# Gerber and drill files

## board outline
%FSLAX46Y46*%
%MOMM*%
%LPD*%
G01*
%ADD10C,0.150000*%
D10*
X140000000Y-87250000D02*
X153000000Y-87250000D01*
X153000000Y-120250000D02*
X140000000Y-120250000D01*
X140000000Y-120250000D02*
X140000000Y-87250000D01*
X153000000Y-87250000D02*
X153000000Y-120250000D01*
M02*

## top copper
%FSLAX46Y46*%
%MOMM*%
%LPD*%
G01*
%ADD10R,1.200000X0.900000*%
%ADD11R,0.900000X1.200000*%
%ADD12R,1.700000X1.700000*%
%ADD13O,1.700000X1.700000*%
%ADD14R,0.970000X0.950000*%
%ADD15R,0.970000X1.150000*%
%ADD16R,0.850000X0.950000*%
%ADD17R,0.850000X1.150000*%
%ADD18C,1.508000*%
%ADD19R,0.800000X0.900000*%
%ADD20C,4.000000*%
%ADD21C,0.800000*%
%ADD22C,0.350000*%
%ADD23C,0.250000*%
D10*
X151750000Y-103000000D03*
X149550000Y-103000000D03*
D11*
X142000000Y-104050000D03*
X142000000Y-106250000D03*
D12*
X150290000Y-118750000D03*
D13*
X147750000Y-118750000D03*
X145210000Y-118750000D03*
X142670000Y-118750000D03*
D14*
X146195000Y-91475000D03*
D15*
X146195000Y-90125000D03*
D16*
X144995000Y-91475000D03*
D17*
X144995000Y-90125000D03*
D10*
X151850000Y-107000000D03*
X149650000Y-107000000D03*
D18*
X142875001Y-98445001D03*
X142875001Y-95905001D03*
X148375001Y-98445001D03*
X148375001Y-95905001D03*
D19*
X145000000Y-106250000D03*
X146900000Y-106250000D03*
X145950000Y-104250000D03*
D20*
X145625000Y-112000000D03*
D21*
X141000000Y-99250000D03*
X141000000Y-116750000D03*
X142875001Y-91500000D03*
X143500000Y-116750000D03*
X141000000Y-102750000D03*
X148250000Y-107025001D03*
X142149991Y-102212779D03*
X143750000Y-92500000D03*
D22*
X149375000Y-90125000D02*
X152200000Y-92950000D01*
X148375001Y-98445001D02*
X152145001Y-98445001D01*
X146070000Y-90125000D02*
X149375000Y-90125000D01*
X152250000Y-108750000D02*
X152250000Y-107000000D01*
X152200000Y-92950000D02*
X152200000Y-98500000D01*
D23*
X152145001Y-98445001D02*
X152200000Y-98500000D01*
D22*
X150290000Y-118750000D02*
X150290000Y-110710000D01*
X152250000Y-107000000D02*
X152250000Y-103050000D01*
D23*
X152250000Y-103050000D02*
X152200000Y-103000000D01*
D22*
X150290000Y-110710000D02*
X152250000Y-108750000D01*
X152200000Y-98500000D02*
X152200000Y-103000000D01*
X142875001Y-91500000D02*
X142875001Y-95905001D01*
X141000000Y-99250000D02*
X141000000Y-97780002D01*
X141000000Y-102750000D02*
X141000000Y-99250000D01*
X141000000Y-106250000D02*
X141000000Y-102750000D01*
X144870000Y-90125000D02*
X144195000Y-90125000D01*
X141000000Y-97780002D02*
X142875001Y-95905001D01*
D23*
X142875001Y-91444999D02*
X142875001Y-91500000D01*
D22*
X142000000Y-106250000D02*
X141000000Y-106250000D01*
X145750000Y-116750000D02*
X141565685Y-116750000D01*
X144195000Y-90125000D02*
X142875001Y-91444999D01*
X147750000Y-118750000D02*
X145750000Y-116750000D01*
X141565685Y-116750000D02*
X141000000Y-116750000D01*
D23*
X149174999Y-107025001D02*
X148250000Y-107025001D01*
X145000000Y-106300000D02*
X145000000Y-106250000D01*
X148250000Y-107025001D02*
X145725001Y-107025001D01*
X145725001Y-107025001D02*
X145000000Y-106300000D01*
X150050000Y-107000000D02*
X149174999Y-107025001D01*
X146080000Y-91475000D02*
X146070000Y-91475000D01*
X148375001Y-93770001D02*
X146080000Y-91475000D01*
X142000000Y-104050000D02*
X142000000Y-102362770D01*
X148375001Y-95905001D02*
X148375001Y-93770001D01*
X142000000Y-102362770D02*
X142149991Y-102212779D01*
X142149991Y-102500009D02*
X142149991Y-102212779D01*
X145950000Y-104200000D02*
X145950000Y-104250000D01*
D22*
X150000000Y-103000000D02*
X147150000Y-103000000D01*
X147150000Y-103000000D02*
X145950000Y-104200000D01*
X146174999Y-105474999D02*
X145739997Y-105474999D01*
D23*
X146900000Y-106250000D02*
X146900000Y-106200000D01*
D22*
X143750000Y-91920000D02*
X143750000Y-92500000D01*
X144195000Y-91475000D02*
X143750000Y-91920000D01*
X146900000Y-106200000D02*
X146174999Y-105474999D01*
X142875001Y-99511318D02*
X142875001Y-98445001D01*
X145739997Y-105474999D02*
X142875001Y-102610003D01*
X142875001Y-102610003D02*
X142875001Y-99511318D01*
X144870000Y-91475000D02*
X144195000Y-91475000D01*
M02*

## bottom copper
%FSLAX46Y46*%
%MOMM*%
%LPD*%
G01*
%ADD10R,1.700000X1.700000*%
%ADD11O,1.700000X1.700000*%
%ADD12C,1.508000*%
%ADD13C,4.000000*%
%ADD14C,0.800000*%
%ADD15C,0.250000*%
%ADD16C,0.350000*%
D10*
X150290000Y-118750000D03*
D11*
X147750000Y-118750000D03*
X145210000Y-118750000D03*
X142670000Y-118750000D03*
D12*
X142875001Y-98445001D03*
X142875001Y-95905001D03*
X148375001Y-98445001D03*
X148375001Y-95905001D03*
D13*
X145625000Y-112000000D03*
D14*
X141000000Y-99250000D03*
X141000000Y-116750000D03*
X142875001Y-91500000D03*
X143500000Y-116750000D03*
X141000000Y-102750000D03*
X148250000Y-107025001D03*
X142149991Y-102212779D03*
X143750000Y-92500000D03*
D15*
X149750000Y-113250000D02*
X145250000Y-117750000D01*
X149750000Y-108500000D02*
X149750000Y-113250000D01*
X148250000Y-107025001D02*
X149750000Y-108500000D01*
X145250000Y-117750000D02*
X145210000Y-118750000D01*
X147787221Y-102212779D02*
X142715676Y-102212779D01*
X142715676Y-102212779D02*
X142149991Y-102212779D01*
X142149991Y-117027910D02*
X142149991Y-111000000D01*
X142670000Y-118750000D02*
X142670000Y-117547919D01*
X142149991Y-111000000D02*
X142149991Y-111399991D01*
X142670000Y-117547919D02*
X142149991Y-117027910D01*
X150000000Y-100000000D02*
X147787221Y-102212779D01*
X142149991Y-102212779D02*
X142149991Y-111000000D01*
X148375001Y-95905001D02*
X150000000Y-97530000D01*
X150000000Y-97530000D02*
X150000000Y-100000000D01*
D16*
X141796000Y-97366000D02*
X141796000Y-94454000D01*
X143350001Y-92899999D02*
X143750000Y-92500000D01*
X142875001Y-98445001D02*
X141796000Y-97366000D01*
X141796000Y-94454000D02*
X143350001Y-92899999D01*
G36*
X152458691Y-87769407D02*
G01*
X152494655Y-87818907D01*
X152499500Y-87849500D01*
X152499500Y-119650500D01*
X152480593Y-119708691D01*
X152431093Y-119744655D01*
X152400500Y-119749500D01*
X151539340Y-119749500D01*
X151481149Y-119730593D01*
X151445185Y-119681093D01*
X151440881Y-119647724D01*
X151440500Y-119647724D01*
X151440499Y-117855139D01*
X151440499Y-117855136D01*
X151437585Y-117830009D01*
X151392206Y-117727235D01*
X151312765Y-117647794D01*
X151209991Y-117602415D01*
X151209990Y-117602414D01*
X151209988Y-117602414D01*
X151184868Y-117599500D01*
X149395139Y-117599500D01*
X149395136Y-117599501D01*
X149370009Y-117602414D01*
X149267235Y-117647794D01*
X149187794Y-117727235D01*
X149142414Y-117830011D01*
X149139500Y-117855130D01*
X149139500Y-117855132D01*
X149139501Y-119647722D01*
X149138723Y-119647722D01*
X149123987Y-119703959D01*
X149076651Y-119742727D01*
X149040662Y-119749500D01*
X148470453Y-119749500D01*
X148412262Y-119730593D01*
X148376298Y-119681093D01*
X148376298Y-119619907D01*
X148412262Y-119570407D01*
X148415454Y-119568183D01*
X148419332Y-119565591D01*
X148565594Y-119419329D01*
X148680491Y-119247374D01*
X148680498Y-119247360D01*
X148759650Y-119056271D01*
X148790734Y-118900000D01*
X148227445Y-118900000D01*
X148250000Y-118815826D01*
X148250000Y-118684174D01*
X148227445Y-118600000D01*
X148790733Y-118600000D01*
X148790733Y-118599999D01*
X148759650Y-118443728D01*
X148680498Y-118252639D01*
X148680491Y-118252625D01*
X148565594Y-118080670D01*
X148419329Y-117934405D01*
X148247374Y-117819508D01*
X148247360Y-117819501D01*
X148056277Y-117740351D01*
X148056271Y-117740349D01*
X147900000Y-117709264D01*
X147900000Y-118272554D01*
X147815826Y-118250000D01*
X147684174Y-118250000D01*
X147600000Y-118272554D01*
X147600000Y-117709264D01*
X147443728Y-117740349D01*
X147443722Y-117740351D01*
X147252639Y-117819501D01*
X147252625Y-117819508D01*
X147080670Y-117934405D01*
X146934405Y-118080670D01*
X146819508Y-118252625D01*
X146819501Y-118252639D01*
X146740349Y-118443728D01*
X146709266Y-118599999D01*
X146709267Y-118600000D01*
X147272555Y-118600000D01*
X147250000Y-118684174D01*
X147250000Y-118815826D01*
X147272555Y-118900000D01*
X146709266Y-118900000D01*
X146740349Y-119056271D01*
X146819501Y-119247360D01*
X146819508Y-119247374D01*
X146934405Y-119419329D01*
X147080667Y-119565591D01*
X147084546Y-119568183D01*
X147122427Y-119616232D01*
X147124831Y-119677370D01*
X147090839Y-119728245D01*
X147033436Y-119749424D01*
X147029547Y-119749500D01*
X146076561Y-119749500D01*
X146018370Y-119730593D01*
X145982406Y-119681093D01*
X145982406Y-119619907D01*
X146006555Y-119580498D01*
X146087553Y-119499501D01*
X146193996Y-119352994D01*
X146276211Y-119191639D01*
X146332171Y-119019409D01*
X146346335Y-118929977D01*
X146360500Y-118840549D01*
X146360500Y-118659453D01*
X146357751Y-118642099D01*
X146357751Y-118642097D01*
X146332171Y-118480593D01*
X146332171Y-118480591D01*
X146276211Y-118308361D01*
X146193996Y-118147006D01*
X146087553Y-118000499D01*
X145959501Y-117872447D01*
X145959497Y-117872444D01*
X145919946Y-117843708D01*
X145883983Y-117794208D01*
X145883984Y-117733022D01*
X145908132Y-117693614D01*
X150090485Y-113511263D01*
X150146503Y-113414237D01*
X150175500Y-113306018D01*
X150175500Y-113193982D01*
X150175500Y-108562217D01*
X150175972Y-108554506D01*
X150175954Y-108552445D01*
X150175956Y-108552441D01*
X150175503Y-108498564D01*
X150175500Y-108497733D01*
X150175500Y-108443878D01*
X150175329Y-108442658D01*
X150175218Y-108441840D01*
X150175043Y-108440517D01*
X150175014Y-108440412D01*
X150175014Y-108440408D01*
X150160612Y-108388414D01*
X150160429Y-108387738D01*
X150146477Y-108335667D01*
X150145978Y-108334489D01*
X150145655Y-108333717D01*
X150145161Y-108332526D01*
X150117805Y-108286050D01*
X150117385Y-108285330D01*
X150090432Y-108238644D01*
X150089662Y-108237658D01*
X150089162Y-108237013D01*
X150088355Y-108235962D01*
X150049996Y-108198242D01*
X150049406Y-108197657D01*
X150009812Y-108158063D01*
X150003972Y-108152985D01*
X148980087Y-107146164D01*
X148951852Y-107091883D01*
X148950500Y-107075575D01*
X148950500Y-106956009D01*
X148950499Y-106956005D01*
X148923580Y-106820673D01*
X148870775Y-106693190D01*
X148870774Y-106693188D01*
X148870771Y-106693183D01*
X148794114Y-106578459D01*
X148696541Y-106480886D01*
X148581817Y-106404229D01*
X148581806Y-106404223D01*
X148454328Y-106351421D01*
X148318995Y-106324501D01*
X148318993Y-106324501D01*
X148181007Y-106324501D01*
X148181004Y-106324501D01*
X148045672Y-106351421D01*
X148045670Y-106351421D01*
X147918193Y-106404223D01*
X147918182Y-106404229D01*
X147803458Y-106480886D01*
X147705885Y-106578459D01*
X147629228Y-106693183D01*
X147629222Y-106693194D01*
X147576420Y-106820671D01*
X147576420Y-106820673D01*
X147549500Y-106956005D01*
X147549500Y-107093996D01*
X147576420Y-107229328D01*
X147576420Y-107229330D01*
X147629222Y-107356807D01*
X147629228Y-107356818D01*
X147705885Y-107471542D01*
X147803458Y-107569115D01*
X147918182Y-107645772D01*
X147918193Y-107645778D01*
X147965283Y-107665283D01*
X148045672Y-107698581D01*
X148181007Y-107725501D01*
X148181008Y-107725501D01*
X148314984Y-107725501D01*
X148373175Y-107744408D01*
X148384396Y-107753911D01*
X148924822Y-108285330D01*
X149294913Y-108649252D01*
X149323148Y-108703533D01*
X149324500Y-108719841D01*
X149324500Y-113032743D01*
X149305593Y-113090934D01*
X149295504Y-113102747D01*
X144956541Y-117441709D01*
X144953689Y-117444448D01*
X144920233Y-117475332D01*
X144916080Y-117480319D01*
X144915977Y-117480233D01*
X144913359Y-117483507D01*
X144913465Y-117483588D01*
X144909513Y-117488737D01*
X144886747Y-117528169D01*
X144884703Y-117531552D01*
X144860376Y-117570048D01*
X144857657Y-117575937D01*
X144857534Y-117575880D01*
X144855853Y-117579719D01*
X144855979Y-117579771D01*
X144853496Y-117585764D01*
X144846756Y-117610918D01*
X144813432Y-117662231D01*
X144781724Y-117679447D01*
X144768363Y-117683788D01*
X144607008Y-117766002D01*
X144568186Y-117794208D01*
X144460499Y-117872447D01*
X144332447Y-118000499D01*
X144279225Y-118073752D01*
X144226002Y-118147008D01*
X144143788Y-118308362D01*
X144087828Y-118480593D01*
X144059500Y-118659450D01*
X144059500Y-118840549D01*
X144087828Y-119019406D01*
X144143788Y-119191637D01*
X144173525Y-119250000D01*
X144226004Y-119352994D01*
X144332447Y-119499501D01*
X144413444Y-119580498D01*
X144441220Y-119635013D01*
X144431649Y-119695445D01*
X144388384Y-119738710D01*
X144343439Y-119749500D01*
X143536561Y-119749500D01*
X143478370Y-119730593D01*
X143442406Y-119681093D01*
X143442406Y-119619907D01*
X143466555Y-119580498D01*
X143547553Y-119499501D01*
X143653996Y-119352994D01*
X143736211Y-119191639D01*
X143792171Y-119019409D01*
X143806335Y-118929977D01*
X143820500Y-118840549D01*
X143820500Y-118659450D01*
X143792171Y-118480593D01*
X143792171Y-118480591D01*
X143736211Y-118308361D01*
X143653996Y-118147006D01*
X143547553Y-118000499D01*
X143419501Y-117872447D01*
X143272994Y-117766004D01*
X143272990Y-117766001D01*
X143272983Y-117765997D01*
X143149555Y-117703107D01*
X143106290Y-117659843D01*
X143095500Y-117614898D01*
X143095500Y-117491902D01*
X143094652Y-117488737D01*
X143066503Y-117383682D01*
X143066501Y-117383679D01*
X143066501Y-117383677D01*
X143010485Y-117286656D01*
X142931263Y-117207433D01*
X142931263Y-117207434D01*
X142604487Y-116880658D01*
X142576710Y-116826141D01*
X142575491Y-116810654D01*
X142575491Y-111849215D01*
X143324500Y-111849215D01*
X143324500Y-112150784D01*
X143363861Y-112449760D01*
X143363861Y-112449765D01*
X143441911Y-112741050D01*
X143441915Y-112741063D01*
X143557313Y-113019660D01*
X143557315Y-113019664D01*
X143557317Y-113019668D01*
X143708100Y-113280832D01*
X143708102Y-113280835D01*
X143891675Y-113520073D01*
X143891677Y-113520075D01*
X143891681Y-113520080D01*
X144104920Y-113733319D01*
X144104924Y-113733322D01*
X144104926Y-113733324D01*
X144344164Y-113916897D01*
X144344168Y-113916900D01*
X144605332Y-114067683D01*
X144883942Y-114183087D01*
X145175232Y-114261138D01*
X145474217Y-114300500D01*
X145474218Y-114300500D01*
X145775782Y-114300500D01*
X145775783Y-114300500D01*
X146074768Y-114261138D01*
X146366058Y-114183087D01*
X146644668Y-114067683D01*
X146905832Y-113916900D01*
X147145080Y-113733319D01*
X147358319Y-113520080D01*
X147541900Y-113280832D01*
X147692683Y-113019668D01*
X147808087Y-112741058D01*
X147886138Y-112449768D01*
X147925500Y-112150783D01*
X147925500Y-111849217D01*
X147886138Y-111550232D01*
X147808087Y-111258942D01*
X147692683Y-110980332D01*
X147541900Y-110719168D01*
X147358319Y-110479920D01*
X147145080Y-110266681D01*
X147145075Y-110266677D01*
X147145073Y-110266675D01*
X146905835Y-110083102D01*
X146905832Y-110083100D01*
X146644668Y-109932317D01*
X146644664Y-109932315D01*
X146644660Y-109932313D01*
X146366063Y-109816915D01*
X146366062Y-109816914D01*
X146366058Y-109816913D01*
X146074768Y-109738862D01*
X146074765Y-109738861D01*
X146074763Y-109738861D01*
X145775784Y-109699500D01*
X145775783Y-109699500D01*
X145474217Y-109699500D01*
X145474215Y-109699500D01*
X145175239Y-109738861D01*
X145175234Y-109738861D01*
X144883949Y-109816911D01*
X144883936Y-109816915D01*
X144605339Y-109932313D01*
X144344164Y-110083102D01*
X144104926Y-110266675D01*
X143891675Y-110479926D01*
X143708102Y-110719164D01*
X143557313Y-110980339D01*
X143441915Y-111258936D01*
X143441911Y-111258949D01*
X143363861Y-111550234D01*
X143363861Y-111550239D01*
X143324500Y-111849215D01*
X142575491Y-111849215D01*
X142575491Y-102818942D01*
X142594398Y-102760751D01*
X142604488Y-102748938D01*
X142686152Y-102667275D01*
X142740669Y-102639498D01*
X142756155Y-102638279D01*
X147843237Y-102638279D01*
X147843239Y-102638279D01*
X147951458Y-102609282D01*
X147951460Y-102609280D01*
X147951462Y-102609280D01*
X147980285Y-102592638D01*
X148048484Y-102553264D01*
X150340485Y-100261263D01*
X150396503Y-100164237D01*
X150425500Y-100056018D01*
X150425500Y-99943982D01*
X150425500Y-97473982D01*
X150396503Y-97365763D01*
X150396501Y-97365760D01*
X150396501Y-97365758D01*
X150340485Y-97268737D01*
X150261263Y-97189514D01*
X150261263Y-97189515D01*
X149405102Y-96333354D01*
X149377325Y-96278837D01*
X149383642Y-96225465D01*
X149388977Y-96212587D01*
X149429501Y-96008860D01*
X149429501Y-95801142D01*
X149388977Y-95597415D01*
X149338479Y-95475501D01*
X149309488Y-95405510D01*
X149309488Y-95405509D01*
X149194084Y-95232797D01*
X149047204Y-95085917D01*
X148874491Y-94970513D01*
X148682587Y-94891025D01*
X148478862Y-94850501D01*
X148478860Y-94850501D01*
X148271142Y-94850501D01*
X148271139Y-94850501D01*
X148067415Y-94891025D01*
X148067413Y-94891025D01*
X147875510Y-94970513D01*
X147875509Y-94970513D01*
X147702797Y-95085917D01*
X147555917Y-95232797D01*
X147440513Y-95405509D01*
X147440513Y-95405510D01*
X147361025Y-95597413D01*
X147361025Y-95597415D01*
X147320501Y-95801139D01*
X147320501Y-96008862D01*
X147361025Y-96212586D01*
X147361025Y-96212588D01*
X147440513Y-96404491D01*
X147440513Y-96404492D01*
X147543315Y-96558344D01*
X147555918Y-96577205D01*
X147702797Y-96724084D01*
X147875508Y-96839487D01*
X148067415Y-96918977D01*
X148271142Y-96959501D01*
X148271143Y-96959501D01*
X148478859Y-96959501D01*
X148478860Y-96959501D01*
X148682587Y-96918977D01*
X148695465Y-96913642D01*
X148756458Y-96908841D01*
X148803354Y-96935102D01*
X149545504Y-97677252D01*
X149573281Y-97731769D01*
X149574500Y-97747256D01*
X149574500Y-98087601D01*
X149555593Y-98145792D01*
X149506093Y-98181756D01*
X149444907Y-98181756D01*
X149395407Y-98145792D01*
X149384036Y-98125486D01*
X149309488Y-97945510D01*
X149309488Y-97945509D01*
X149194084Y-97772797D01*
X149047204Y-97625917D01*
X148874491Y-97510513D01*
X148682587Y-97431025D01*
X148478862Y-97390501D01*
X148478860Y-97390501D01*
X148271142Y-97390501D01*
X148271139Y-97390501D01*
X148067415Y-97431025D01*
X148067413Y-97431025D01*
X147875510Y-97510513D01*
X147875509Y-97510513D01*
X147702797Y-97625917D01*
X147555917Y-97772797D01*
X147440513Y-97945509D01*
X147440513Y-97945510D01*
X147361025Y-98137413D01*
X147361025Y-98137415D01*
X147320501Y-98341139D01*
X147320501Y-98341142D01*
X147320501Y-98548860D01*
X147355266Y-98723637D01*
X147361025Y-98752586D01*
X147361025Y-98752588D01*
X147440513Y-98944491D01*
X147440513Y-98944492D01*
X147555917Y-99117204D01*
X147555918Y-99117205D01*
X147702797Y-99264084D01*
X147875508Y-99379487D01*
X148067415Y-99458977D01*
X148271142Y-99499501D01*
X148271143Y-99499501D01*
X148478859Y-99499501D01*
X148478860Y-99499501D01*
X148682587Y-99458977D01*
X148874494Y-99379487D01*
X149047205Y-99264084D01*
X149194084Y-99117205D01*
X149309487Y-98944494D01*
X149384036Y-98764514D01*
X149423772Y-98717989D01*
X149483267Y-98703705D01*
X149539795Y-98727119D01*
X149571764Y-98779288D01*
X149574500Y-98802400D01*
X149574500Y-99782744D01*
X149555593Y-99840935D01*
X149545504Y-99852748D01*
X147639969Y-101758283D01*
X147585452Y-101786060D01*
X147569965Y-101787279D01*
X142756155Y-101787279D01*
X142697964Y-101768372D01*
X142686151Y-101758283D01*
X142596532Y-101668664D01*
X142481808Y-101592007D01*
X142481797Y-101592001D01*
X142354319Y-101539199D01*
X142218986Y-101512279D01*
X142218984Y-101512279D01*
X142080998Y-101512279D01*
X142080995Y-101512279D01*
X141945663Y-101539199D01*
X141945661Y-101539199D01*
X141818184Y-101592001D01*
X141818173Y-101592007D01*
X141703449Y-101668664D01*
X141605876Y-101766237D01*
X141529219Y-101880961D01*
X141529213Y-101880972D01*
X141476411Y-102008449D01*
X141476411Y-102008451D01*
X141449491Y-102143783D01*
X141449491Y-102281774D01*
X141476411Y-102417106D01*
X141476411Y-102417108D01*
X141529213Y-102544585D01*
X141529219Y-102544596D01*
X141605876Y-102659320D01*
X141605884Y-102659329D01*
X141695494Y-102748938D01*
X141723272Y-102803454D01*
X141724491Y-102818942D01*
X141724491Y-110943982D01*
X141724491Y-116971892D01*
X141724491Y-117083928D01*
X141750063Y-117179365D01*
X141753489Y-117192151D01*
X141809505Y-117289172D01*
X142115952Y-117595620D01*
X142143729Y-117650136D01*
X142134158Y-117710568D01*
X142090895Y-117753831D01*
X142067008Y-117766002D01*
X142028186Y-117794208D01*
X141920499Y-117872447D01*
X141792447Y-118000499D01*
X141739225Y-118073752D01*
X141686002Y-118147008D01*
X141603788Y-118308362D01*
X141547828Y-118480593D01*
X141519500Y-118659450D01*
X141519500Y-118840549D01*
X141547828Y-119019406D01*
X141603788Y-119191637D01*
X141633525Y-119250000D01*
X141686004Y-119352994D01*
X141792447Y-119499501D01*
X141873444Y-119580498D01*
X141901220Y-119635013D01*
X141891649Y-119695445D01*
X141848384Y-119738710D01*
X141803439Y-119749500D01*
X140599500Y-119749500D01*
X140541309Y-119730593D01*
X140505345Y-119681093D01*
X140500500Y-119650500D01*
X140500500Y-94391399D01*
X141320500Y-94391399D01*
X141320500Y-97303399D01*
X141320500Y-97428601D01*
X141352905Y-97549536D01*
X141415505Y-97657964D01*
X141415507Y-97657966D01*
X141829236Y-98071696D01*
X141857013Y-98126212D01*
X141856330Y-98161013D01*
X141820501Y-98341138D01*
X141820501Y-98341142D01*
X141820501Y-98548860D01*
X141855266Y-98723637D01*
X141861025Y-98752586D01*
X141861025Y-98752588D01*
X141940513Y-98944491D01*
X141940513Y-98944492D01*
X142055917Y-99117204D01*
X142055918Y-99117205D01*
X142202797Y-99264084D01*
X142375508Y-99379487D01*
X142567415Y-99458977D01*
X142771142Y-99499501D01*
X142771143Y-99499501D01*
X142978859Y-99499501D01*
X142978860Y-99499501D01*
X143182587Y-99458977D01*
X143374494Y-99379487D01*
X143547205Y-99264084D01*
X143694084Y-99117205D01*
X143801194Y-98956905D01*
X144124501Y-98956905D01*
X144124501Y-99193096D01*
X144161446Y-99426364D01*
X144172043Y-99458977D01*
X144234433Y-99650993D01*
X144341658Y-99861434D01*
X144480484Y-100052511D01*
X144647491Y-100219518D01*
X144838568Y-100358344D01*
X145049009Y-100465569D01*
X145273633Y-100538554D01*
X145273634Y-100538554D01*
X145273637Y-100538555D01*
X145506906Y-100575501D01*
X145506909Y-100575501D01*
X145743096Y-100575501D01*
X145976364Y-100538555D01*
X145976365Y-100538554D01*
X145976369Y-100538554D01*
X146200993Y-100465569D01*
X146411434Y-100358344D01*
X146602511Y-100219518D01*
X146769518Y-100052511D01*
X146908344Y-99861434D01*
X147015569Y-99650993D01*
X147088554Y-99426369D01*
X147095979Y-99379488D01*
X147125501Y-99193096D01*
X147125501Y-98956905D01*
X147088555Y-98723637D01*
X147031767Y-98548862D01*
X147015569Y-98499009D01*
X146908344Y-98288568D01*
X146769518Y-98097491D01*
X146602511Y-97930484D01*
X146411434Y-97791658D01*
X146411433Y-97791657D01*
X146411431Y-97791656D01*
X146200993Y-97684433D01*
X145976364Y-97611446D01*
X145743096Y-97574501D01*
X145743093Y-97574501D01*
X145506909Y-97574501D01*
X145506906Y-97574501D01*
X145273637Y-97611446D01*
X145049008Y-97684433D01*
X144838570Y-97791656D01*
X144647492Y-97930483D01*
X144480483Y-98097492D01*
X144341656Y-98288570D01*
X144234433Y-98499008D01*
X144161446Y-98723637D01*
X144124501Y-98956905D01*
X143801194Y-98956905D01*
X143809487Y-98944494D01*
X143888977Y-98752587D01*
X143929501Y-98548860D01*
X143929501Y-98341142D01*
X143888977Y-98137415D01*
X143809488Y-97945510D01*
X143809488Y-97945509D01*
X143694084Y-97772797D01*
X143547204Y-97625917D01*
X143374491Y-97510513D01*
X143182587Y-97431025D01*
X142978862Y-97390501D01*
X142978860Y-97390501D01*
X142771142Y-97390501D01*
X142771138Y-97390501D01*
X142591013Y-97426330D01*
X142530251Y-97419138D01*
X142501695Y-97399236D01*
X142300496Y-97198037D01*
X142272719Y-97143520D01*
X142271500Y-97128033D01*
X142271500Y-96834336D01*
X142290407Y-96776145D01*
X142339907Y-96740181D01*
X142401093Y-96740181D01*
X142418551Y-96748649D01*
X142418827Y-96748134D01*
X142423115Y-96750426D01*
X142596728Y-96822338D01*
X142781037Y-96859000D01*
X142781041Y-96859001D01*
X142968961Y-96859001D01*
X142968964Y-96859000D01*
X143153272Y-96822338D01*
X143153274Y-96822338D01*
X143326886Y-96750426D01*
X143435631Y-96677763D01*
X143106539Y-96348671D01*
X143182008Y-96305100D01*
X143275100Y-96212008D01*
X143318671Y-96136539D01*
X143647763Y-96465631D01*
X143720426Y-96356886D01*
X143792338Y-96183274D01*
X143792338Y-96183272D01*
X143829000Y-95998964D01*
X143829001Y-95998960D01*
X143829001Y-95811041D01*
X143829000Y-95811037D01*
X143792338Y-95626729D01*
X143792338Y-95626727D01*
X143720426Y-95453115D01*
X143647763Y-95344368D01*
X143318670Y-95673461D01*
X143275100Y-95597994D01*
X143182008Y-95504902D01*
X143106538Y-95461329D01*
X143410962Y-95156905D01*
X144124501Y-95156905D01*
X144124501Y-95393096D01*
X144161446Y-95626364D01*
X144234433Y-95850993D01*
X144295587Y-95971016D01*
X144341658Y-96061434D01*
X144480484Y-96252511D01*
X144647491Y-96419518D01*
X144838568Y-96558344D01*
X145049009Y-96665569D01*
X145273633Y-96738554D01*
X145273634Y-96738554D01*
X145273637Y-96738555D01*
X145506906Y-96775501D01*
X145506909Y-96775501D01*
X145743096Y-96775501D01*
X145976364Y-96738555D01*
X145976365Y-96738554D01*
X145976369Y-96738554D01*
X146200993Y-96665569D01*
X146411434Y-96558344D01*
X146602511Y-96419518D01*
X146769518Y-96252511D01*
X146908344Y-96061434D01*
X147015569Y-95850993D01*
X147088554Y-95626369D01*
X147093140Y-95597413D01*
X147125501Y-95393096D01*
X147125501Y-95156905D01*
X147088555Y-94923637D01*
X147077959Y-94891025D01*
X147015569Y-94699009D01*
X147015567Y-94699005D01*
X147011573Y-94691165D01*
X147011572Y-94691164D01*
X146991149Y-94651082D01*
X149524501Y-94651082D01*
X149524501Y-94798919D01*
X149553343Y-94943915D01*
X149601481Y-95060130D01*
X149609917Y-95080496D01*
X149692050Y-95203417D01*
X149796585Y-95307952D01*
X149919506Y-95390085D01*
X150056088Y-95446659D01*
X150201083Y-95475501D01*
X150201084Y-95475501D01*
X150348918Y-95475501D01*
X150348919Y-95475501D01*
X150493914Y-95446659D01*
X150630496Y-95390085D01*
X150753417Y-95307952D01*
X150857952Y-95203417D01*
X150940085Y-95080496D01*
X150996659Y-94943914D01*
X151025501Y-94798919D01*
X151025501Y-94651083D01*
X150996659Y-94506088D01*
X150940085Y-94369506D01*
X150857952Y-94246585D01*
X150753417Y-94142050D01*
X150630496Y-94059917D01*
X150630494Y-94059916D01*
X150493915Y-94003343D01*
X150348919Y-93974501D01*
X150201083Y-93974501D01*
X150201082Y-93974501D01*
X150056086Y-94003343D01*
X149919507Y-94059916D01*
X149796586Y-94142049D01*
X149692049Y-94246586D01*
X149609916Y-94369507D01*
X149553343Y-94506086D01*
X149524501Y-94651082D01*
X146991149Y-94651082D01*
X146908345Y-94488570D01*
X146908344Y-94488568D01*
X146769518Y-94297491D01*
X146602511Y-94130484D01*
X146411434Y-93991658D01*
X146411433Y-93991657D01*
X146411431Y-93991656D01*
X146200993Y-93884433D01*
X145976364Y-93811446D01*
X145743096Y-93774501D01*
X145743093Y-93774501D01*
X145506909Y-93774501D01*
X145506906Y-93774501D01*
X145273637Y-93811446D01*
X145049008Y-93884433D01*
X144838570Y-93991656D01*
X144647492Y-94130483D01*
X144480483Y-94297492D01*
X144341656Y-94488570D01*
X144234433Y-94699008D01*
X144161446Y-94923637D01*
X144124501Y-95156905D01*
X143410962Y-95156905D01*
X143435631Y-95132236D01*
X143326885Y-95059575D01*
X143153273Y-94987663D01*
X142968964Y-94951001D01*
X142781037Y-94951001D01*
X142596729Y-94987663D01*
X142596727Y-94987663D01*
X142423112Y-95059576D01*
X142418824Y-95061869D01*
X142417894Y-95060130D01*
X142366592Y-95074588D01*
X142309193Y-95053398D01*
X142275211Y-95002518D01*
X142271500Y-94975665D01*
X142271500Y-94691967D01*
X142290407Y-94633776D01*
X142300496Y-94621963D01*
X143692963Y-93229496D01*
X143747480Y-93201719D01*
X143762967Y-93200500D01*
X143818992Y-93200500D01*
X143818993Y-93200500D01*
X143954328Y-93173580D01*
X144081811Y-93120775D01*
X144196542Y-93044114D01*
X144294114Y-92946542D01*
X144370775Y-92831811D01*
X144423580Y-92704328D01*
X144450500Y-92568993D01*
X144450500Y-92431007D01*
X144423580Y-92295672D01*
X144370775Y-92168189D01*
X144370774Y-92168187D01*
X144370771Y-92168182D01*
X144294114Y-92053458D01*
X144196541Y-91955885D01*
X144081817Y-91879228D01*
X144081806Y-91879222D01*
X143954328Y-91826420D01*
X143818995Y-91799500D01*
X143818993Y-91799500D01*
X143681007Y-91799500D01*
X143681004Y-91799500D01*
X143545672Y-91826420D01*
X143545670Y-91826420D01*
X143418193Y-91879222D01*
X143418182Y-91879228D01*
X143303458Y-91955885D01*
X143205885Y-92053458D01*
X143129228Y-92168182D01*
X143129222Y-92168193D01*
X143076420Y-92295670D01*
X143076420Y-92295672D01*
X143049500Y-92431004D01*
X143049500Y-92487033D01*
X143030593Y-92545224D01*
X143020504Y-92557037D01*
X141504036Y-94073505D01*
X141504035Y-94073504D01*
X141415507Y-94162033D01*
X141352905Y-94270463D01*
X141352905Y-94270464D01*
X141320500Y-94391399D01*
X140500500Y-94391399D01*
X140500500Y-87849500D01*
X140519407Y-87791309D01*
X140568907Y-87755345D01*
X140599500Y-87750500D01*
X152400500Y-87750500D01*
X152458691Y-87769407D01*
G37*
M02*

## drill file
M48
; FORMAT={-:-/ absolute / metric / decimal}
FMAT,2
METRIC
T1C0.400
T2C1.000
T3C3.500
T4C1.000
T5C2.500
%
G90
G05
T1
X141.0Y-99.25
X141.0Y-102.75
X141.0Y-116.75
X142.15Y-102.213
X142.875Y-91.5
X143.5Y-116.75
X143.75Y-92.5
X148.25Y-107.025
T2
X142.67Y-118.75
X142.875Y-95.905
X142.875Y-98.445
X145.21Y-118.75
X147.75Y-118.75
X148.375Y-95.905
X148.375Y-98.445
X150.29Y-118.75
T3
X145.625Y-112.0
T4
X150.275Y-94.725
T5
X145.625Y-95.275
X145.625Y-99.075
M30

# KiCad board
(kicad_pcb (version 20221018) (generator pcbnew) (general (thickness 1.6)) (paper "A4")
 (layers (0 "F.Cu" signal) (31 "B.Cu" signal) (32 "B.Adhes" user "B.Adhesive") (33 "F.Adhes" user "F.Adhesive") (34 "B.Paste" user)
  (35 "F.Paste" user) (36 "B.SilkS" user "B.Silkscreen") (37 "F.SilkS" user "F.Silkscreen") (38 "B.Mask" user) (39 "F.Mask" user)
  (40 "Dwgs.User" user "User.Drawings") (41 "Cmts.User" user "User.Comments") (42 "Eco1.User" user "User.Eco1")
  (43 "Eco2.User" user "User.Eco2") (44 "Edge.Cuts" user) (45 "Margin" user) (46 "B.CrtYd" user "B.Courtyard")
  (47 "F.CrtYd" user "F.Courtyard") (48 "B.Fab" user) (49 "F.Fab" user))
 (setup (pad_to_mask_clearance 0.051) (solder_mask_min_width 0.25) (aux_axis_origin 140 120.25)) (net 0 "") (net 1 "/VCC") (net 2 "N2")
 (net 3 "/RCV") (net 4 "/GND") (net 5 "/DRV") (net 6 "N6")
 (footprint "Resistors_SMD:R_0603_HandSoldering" (layer "F.Cu") (at 150.65 103 180)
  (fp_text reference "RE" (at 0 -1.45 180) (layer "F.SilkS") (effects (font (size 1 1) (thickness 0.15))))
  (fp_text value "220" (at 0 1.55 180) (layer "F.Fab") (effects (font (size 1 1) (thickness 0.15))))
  (pad "1" smd rect (at -1.1 0 180) (size 1.2 0.9) (layers "F.Cu" "F.Paste" "F.Mask") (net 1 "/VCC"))
  (pad "2" smd rect (at 1.1 0 180) (size 1.2 0.9) (layers "F.Cu" "F.Paste" "F.Mask") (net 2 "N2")))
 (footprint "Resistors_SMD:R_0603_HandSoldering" (layer "F.Cu") (at 142 105.15 -90)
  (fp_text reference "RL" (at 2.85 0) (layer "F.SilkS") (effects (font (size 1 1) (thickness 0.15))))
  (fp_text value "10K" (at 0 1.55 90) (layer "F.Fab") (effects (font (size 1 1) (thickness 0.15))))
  (pad "1" smd rect (at -1.1 0 270) (size 1.2 0.9) (layers "F.Cu" "F.Paste" "F.Mask") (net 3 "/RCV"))
  (pad "2" smd rect (at 1.1 0 270) (size 1.2 0.9) (layers "F.Cu" "F.Paste" "F.Mask") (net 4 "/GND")))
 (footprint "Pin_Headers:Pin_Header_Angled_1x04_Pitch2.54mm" (layer "F.Cu") (at 150.29 118.75 -90)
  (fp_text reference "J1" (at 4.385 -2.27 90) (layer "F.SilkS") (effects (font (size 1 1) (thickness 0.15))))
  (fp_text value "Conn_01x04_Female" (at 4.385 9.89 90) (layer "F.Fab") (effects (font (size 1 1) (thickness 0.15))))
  (pad "1" thru_hole rect (at 0 0 270) (size 1.7 1.7) (drill 1) (layers "*.Cu" "*.Mask") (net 1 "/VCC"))
  (pad "2" thru_hole oval (at 0 2.54 270) (size 1.7 1.7) (drill 1) (layers "*.Cu" "*.Mask") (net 4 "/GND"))
  (pad "3" thru_hole oval (at 0 5.08 270) (size 1.7 1.7) (drill 1) (layers "*.Cu" "*.Mask") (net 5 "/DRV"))
  (pad "4" thru_hole oval (at 0 7.62 270) (size 1.7 1.7) (drill 1) (layers "*.Cu" "*.Mask") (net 3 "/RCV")))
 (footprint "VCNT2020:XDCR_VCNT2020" (layer "F.Cu") (at 145.625 90.75 180)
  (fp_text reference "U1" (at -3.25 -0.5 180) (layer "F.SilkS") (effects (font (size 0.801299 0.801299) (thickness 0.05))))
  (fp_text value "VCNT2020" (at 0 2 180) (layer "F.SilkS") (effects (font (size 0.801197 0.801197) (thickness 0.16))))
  (pad "1" smd rect (at -0.57 -0.725 180) (size 0.97 0.95) (layers "F.Cu" "F.Paste" "F.Mask") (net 3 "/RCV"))
  (pad "2" smd rect (at -0.57 0.625 180) (size 0.97 1.15) (layers "F.Cu" "F.Paste" "F.Mask") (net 1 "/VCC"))
  (pad "3" smd rect (at 0.63 -0.725 180) (size 0.85 0.95) (layers "F.Cu" "F.Paste" "F.Mask") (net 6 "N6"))
  (pad "4" smd rect (at 0.63 0.625 180) (size 0.85 1.15) (layers "F.Cu" "F.Paste" "F.Mask") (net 4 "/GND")))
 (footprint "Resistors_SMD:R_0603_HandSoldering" (layer "F.Cu") (at 150.75 107 180)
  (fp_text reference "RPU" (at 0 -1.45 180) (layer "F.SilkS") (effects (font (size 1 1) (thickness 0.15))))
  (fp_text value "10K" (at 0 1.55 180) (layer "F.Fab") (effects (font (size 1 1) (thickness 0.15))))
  (pad "1" smd rect (at -1.1 0 180) (size 1.2 0.9) (layers "F.Cu" "F.Paste" "F.Mask") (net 1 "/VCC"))
  (pad "2" smd rect (at 1.1 0 180) (size 1.2 0.9) (layers "F.Cu" "F.Paste" "F.Mask") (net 5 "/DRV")))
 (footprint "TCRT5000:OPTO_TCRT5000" (layer "F.Cu") (at 145.625001 97.175001 180)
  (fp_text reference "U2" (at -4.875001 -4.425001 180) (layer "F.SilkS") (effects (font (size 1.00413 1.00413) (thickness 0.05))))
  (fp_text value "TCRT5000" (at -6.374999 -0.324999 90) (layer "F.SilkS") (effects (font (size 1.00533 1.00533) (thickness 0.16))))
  (pad "" np_thru_hole circle (at -4.65 2.45 180) (size 1 1) (drill 1) (layers "*.Cu" "*.Mask" "F.SilkS"))
  (pad "" np_thru_hole circle (at 0 -1.9 180) (size 2.5 2.5) (drill 2.5) (layers "*.Cu" "*.Mask" "F.SilkS"))
  (pad "" np_thru_hole circle (at 0 1.9 180) (size 2.5 2.5) (drill 2.5) (layers "*.Cu" "*.Mask" "F.SilkS"))
  (pad "A" thru_hole circle (at 2.75 -1.27 180) (size 1.508 1.508) (drill 1) (layers "*.Cu" "*.Mask") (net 6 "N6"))
  (pad "CATH" thru_hole circle (at 2.75 1.27 180) (size 1.508 1.508) (drill 1) (layers "*.Cu" "*.Mask") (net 4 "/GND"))
  (pad "COLL" thru_hole circle (at -2.75 -1.27 180) (size 1.508 1.508) (drill 1) (layers "*.Cu" "*.Mask") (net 1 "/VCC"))
  (pad "E" thru_hole circle (at -2.75 1.27 180) (size 1.508 1.508) (drill 1) (layers "*.Cu" "*.Mask") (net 3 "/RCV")))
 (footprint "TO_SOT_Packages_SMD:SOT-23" (layer "F.Cu") (at 145.95 105.25 90)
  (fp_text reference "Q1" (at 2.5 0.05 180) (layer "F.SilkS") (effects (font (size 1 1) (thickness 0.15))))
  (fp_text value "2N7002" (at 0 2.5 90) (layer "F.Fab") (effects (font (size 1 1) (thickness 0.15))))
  (pad "1" smd rect (at -1 -0.95 90) (size 0.9 0.8) (layers "F.Cu" "F.Paste" "F.Mask") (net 5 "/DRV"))
  (pad "2" smd rect (at -1 0.95 90) (size 0.9 0.8) (layers "F.Cu" "F.Paste" "F.Mask") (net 6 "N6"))
  (pad "3" smd rect (at 1 0 90) (size 0.9 0.8) (layers "F.Cu" "F.Paste" "F.Mask") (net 2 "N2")))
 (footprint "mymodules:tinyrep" (layer "B.Cu") (at 151.25 109.5 -90)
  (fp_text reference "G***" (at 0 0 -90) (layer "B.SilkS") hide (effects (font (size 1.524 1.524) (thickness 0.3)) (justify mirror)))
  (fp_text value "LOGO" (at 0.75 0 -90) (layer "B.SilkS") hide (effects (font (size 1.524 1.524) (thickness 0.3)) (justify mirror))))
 (gr_line (start 140 87.25) (end 153 87.25) (stroke (width 0.15) (type solid)) (layer "Edge.Cuts"))
 (gr_line (start 153 120.25) (end 140 120.25) (stroke (width 0.15) (type solid)) (layer "Edge.Cuts"))
 (gr_line (start 140 120.25) (end 140 87.25) (stroke (width 0.15) (type solid)) (layer "Edge.Cuts"))
 (gr_line (start 153 87.25) (end 153 120.25) (stroke (width 0.15) (type solid)) (layer "Edge.Cuts"))
 (via (at 145.625 112) (size 4) (drill 3.5) (layers "F.Cu" "B.Cu") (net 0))
 (segment (start 149.375 90.125) (end 152.2 92.95) (width 0.35) (layer "F.Cu") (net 1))
 (segment (start 148.375001 98.445001) (end 152.145001 98.445001) (width 0.35) (layer "F.Cu") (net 1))
 (segment (start 146.07 90.125) (end 149.375 90.125) (width 0.35) (layer "F.Cu") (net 1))
 (segment (start 152.25 108.75) (end 152.25 107) (width 0.35) (layer "F.Cu") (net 1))
 (segment (start 152.2 92.95) (end 152.2 98.5) (width 0.35) (layer "F.Cu") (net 1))
 (segment (start 152.145001 98.445001) (end 152.2 98.5) (width 0.25) (layer "F.Cu") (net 1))
 (segment (start 150.29 118.75) (end 150.29 110.71) (width 0.35) (layer "F.Cu") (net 1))
 (segment (start 152.25 107) (end 152.25 103.05) (width 0.35) (layer "F.Cu") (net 1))
 (segment (start 152.25 103.05) (end 152.2 103) (width 0.25) (layer "F.Cu") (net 1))
 (segment (start 150.29 110.71) (end 152.25 108.75) (width 0.35) (layer "F.Cu") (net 1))
 (segment (start 152.2 98.5) (end 152.2 103) (width 0.35) (layer "F.Cu") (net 1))
 (segment (start 142.875001 91.5) (end 142.875001 95.905001) (width 0.35) (layer "F.Cu") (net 4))
 (segment (start 141 99.25) (end 141 97.780002) (width 0.35) (layer "F.Cu") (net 4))
 (segment (start 141 102.75) (end 141 99.25) (width 0.35) (layer "F.Cu") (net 4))
 (segment (start 141 106.25) (end 141 102.75) (width 0.35) (layer "F.Cu") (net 4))
 (segment (start 144.87 90.125) (end 144.195 90.125) (width 0.35) (layer "F.Cu") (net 4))
 (segment (start 141 97.780002) (end 142.875001 95.905001) (width 0.35) (layer "F.Cu") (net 4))
 (segment (start 142.875001 91.444999) (end 142.875001 91.5) (width 0.25) (layer "F.Cu") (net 4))
 (segment (start 142 106.25) (end 141 106.25) (width 0.35) (layer "F.Cu") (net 4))
 (segment (start 145.75 116.75) (end 141.565685 116.75) (width 0.35) (layer "F.Cu") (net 4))
 (segment (start 144.195 90.125) (end 142.875001 91.444999) (width 0.35) (layer "F.Cu") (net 4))
 (segment (start 147.75 118.75) (end 145.75 116.75) (width 0.35) (layer "F.Cu") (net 4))
 (segment (start 141.565685 116.75) (end 141 116.75) (width 0.35) (layer "F.Cu") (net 4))
 (via (at 141 99.25) (size 0.8) (drill 0.4) (layers "F.Cu" "B.Cu") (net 4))
 (via (at 141 116.75) (size 0.8) (drill 0.4) (layers "F.Cu" "B.Cu") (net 4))
 (via (at 142.875001 91.5) (size 0.8) (drill 0.4) (layers "F.Cu" "B.Cu") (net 4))
 (via (at 143.5 116.75) (size 0.8) (drill 0.4) (layers "F.Cu" "B.Cu") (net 4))
 (via (at 141 102.75) (size 0.8) (drill 0.4) (layers "F.Cu" "B.Cu") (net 4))
 (segment (start 149.174999 107.025001) (end 148.25 107.025001) (width 0.25) (layer "F.Cu") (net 5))
 (segment (start 145 106.3) (end 145 106.25) (width 0.25) (layer "F.Cu") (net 5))
 (segment (start 148.25 107.025001) (end 145.725001 107.025001) (width 0.25) (layer "F.Cu") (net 5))
 (segment (start 145.725001 107.025001) (end 145 106.3) (width 0.25) (layer "F.Cu") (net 5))
 (segment (start 150.05 107) (end 149.174999 107.025001) (width 0.25) (layer "F.Cu") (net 5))
 (via (at 148.25 107.025001) (size 0.8) (drill 0.4) (layers "F.Cu" "B.Cu") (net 5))
 (segment (start 149.75 113.25) (end 145.25 117.75) (width 0.25) (layer "B.Cu") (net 5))
 (segment (start 149.75 108.5) (end 149.75 113.25) (width 0.25) (layer "B.Cu") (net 5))
 (segment (start 148.25 107.025001) (end 149.75 108.5) (width 0.25) (layer "B.Cu") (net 5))
 (segment (start 145.25 117.75) (end 145.21 118.75) (width 0.25) (layer "B.Cu") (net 5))
 (segment (start 146.08 91.475) (end 146.07 91.475) (width 0.25) (layer "F.Cu") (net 3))
 (segment (start 148.375001 93.770001) (end 146.08 91.475) (width 0.25) (layer "F.Cu") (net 3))
 (segment (start 142 104.05) (end 142 102.36277) (width 0.25) (layer "F.Cu") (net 3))
 (segment (start 148.375001 95.905001) (end 148.375001 93.770001) (width 0.25) (layer "F.Cu") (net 3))
 (segment (start 142 102.36277) (end 142.149991 102.212779) (width 0.25) (layer "F.Cu") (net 3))
 (segment (start 142.149991 102.500009) (end 142.149991 102.212779) (width 0.25) (layer "F.Cu") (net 3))
 (via (at 142.149991 102.212779) (size 0.8) (drill 0.4) (layers "F.Cu" "B.Cu") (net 3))
 (segment (start 147.787221 102.212779) (end 142.715676 102.212779) (width 0.25) (layer "B.Cu") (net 3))
 (segment (start 142.715676 102.212779) (end 142.149991 102.212779) (width 0.25) (layer "B.Cu") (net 3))
 (segment (start 142.149991 117.02791) (end 142.149991 111) (width 0.25) (layer "B.Cu") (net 3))
 (segment (start 142.67 118.75) (end 142.67 117.547919) (width 0.25) (layer "B.Cu") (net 3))
 (segment (start 142.149991 111) (end 142.149991 111.399991) (width 0.25) (layer "B.Cu") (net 3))
 (segment (start 142.67 117.547919) (end 142.149991 117.02791) (width 0.25) (layer "B.Cu") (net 3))
 (segment (start 150 100) (end 147.787221 102.212779) (width 0.25) (layer "B.Cu") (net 3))
 (segment (start 142.149991 102.212779) (end 142.149991 111) (width 0.25) (layer "B.Cu") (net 3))
 (segment (start 148.375001 95.905001) (end 150 97.53) (width 0.25) (layer "B.Cu") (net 3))
 (segment (start 150 97.53) (end 150 100) (width 0.25) (layer "B.Cu") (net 3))
 (segment (start 145.95 104.2) (end 145.95 104.25) (width 0.25) (layer "F.Cu") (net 2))
 (segment (start 150 103) (end 147.15 103) (width 0.35) (layer "F.Cu") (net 2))
 (segment (start 147.15 103) (end 145.95 104.2) (width 0.35) (layer "F.Cu") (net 2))
 (segment (start 146.174999 105.474999) (end 145.739997 105.474999) (width 0.35) (layer "F.Cu") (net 6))
 (segment (start 146.9 106.25) (end 146.9 106.2) (width 0.25) (layer "F.Cu") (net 6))
 (segment (start 143.75 91.92) (end 143.75 92.5) (width 0.35) (layer "F.Cu") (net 6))
 (segment (start 144.195 91.475) (end 143.75 91.92) (width 0.35) (layer "F.Cu") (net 6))
 (segment (start 146.9 106.2) (end 146.174999 105.474999) (width 0.35) (layer "F.Cu") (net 6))
 (segment (start 142.875001 99.511318) (end 142.875001 98.445001) (width 0.35) (layer "F.Cu") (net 6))
 (segment (start 145.739997 105.474999) (end 142.875001 102.610003) (width 0.35) (layer "F.Cu") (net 6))
 (segment (start 142.875001 102.610003) (end 142.875001 99.511318) (width 0.35) (layer "F.Cu") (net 6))
 (segment (start 144.87 91.475) (end 144.195 91.475) (width 0.35) (layer "F.Cu") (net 6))
 (via (at 143.75 92.5) (size 0.8) (drill 0.4) (layers "F.Cu" "B.Cu") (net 6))
 (segment (start 141.796 97.366) (end 141.796 94.454) (width 0.35) (layer "B.Cu") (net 6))
 (segment (start 143.350001 92.899999) (end 143.75 92.5) (width 0.35) (layer "B.Cu") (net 6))
 (segment (start 142.875001 98.445001) (end 141.796 97.366) (width 0.35) (layer "B.Cu") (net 6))
 (segment (start 141.796 94.454) (end 143.350001 92.899999) (width 0.35) (layer "B.Cu") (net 6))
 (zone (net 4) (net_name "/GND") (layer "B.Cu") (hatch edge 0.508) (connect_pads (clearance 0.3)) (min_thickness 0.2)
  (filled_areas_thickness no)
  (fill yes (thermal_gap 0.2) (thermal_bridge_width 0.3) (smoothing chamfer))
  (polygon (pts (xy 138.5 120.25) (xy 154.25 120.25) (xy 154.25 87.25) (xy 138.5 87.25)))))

